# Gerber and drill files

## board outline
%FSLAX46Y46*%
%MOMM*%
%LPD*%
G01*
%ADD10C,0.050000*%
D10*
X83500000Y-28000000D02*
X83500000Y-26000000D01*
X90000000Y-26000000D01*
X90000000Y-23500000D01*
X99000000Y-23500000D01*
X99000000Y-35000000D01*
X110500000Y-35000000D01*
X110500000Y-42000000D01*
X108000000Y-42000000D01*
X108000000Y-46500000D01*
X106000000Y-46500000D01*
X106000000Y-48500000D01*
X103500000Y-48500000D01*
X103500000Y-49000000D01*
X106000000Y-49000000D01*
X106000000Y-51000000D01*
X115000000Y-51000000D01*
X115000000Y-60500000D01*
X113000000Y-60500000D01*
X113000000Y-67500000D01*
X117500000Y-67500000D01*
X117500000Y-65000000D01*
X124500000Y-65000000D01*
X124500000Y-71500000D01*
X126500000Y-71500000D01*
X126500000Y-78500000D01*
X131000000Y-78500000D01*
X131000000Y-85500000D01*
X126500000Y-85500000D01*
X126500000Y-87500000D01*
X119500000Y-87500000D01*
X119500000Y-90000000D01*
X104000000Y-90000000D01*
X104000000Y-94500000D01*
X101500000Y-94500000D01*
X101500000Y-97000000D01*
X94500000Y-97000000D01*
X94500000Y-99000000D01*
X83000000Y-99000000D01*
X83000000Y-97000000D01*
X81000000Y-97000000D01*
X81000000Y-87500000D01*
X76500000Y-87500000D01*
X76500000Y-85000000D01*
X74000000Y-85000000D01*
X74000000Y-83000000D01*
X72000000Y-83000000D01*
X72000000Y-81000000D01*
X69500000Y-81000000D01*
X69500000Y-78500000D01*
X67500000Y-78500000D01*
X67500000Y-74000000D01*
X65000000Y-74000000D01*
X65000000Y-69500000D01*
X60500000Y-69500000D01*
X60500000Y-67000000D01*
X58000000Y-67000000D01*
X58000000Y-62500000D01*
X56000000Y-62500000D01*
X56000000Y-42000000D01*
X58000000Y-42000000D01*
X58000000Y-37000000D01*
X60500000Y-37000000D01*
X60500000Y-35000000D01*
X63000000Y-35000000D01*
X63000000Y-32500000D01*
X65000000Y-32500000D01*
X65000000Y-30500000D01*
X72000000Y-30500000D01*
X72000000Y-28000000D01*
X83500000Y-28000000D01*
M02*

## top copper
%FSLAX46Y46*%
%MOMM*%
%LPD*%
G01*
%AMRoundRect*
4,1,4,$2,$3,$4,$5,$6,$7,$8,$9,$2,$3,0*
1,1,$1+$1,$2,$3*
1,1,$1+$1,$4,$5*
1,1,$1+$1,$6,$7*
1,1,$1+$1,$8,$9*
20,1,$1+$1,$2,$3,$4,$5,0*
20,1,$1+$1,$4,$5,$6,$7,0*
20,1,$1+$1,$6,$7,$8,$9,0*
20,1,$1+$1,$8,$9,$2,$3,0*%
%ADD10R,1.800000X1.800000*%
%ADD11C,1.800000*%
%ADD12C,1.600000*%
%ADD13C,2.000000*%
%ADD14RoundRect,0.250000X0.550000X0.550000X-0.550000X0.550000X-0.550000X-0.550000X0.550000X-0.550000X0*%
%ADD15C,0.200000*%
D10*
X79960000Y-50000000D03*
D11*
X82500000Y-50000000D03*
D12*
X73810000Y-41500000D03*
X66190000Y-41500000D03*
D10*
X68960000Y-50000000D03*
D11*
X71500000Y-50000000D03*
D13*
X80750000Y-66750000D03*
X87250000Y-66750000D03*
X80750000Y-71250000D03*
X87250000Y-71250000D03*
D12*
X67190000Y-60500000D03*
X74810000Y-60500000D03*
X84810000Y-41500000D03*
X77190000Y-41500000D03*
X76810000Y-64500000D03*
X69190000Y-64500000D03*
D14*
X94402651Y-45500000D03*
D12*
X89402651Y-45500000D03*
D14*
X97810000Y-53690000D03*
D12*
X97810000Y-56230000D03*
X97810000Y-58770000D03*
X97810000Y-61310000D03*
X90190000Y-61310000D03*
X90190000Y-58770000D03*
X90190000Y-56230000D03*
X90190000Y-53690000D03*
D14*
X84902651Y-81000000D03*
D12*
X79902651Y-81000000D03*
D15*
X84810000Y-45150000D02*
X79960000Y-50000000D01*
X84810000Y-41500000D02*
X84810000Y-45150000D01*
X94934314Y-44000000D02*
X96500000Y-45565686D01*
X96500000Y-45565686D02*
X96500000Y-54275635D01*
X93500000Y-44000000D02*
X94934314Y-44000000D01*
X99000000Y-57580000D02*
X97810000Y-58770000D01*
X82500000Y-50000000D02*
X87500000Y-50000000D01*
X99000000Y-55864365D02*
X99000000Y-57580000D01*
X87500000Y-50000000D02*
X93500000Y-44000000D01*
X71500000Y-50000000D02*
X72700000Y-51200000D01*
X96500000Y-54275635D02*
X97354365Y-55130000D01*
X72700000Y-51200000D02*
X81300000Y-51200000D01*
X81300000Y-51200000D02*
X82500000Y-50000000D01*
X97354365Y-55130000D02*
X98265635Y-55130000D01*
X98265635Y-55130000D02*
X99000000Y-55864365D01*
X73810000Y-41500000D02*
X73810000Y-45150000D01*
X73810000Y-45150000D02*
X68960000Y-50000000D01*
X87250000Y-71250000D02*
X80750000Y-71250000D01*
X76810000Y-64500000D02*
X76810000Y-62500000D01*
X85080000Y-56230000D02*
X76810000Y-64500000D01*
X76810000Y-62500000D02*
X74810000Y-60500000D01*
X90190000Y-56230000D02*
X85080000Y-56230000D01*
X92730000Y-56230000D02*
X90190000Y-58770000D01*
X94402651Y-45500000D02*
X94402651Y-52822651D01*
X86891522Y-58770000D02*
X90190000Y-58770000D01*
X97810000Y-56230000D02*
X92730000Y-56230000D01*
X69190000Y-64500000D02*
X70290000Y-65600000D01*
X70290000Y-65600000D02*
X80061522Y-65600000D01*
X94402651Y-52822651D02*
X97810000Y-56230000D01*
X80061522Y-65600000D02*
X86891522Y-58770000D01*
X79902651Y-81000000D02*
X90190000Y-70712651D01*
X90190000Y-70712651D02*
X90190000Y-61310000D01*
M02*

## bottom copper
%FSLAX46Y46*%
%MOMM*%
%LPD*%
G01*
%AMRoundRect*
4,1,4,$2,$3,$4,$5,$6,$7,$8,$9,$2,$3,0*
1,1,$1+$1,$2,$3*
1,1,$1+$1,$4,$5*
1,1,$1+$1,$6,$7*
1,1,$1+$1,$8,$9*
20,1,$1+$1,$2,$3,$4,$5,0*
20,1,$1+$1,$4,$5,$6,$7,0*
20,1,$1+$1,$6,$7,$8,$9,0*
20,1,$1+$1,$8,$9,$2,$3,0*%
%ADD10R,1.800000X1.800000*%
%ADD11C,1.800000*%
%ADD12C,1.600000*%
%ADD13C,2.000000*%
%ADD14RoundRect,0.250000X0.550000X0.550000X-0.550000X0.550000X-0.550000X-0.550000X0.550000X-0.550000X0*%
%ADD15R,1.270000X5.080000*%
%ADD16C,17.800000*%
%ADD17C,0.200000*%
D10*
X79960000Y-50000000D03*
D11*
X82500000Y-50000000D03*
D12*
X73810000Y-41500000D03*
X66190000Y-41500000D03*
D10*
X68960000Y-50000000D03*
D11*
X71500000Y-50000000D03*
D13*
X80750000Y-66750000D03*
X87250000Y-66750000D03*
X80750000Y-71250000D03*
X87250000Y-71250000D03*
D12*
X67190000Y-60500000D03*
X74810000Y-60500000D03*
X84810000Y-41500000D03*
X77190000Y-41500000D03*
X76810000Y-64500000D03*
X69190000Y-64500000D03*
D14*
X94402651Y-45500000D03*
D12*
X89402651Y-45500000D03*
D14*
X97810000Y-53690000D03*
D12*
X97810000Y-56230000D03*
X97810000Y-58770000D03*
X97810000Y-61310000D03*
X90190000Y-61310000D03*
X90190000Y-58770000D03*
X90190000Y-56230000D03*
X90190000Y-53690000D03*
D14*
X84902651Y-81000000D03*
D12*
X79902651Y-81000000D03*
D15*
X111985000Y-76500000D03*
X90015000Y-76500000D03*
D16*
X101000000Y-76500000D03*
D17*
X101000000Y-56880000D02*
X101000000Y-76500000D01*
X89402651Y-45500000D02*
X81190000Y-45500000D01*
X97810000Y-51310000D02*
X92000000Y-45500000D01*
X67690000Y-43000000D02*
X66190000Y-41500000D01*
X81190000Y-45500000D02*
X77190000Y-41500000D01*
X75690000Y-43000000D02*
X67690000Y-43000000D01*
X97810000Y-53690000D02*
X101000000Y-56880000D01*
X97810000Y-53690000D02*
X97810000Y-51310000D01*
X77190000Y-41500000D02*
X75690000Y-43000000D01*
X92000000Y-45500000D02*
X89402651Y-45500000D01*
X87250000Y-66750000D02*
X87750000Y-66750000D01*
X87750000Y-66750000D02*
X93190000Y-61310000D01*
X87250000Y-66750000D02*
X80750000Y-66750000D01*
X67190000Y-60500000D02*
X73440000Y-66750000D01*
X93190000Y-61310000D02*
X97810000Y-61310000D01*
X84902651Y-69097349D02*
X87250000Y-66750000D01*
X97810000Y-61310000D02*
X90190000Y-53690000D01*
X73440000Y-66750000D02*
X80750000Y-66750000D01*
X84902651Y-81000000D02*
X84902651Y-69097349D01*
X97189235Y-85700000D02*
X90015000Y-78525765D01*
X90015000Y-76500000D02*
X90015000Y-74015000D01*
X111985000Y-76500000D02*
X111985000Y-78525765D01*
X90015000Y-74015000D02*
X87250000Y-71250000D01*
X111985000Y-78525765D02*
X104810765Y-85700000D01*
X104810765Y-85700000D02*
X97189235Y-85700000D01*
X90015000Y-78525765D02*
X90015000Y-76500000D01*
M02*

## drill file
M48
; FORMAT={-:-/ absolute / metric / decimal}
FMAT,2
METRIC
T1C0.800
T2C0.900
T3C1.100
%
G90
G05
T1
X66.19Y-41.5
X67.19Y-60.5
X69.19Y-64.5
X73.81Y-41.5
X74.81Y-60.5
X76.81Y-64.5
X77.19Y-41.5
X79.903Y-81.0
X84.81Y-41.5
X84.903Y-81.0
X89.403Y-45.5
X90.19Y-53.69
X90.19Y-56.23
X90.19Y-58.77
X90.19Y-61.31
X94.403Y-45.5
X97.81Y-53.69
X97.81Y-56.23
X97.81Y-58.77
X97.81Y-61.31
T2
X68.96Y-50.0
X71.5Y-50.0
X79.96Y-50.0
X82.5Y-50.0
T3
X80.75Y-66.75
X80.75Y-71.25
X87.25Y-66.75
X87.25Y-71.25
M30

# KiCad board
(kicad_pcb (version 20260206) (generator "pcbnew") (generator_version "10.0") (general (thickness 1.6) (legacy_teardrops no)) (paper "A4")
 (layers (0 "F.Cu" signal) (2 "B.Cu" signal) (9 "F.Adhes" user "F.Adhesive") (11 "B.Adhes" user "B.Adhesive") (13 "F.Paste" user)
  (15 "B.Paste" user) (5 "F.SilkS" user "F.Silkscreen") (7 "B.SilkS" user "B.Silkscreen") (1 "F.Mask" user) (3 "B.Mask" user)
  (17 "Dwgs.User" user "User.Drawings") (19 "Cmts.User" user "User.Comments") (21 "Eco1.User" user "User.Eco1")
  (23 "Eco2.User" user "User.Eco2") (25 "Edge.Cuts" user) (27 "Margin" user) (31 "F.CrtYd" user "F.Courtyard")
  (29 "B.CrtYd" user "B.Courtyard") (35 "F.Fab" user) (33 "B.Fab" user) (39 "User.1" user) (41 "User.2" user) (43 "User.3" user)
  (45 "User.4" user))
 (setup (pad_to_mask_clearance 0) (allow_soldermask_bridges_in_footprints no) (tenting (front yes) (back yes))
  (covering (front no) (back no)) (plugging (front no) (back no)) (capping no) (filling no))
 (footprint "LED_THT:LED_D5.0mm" (layer "F.Cu") (at 79.96 50)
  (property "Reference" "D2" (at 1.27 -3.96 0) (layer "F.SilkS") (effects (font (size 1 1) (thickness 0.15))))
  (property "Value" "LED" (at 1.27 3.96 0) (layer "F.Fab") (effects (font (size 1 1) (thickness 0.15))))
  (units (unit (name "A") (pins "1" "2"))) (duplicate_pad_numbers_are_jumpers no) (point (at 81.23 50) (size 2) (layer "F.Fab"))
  (pad "1" thru_hole rect (at 0 0) (size 1.8 1.8) (drill 0.9) (layers "*.Cu" "*.Mask") (remove_unused_layers no) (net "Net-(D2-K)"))
  (pad "2" thru_hole circle (at 2.54 0) (size 1.8 1.8) (drill 0.9) (layers "*.Cu" "*.Mask") (remove_unused_layers no) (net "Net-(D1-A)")))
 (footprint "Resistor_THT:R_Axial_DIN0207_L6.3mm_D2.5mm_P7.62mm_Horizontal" (layer "F.Cu") (at 73.81 41.5 180)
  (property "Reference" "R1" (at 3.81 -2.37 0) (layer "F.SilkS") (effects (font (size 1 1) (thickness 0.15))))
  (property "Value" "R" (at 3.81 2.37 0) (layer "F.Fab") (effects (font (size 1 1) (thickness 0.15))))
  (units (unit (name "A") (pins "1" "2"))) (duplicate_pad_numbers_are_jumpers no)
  (pad "1" thru_hole circle (at 0 0 180) (size 1.6 1.6) (drill 0.8) (layers "*.Cu" "*.Mask") (remove_unused_layers no) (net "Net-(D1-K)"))
  (pad "2" thru_hole circle (at 7.62 0 180) (size 1.6 1.6) (drill 0.8) (layers "*.Cu" "*.Mask") (remove_unused_layers no)
   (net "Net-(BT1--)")))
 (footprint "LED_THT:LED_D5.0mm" (layer "F.Cu") (at 68.96 50)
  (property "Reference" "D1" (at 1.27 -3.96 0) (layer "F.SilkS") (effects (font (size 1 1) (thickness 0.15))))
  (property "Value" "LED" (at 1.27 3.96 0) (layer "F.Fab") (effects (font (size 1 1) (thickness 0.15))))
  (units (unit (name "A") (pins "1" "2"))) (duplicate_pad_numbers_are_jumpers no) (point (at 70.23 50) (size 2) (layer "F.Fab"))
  (pad "1" thru_hole rect (at 0 0) (size 1.8 1.8) (drill 0.9) (layers "*.Cu" "*.Mask") (remove_unused_layers no) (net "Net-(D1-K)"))
  (pad "2" thru_hole circle (at 2.54 0) (size 1.8 1.8) (drill 0.9) (layers "*.Cu" "*.Mask") (remove_unused_layers no) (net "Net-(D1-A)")))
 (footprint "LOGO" (layer "F.Cu") (at 93.5 61.5)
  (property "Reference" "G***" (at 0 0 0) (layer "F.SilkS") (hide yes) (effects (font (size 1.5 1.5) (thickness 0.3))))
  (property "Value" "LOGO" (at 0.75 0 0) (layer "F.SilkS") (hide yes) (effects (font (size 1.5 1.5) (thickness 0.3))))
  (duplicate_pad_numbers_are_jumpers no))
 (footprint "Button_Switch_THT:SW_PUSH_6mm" (layer "F.Cu") (at 80.75 66.75)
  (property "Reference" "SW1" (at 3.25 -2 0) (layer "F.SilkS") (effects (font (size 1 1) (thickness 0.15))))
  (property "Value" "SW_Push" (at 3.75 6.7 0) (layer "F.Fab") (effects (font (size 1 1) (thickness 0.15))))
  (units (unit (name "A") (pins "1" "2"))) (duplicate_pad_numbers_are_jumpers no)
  (pad "1" thru_hole circle (at 0 0 90) (size 2 2) (drill 1.1) (layers "*.Cu" "*.Mask") (remove_unused_layers no) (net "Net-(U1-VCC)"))
  (pad "1" thru_hole circle (at 6.5 0 90) (size 2 2) (drill 1.1) (layers "*.Cu" "*.Mask") (remove_unused_layers no) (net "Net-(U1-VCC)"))
  (pad "2" thru_hole circle (at 0 4.5 90) (size 2 2) (drill 1.1) (layers "*.Cu" "*.Mask") (remove_unused_layers no) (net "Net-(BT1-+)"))
  (pad "2" thru_hole circle (at 6.5 4.5 90) (size 2 2) (drill 1.1) (layers "*.Cu" "*.Mask") (remove_unused_layers no) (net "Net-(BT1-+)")))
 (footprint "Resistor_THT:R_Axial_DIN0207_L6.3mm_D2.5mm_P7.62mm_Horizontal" (layer "F.Cu") (at 67.19 60.5)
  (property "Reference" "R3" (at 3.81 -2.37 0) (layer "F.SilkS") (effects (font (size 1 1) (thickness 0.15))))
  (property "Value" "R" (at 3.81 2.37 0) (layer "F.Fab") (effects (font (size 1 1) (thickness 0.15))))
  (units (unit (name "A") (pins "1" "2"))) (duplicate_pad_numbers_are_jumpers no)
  (pad "1" thru_hole circle (at 0 0) (size 1.6 1.6) (drill 0.8) (layers "*.Cu" "*.Mask") (remove_unused_layers no) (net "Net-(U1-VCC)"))
  (pad "2" thru_hole circle (at 7.62 0) (size 1.6 1.6) (drill 0.8) (layers "*.Cu" "*.Mask") (remove_unused_layers no) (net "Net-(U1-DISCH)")))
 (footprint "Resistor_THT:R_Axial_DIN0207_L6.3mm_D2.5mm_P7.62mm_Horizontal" (layer "F.Cu") (at 84.81 41.5 180)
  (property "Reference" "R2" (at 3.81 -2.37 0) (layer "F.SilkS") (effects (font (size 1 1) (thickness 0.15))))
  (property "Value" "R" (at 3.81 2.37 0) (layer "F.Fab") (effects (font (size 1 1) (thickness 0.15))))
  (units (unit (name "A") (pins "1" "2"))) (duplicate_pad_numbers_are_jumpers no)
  (pad "1" thru_hole circle (at 0 0 180) (size 1.6 1.6) (drill 0.8) (layers "*.Cu" "*.Mask") (remove_unused_layers no) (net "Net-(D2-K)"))
  (pad "2" thru_hole circle (at 7.62 0 180) (size 1.6 1.6) (drill 0.8) (layers "*.Cu" "*.Mask") (remove_unused_layers no)
   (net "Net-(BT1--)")))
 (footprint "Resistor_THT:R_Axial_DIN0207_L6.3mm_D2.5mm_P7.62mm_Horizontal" (layer "B.Cu") (at 76.81 64.5 180)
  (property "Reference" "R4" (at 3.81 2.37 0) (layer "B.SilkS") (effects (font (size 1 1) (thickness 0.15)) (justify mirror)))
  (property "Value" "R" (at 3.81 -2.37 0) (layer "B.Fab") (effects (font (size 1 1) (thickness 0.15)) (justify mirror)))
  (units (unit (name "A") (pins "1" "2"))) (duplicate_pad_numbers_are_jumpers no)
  (pad "1" thru_hole circle (at 0 0 180) (size 1.6 1.6) (drill 0.8) (layers "*.Cu" "*.Mask") (remove_unused_layers no)
   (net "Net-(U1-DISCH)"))
  (pad "2" thru_hole circle (at 7.62 0 180) (size 1.6 1.6) (drill 0.8) (layers "*.Cu" "*.Mask") (remove_unused_layers no)
   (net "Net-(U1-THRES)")))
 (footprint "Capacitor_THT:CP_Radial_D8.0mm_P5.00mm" (layer "B.Cu") (at 94.402651 45.5 180)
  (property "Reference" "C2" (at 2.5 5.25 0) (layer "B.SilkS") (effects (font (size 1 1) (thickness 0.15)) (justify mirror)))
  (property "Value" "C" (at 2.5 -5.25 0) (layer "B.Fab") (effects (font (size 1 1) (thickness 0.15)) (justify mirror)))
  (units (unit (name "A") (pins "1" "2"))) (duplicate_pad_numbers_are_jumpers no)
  (pad "1" thru_hole roundrect (at 0 0 180) (size 1.6 1.6) (drill 0.8) (layers "*.Cu" "*.Mask") (remove_unused_layers no)
   (roundrect_rratio 0.15625) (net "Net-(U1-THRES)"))
  (pad "2" thru_hole circle (at 5 0 180) (size 1.6 1.6) (drill 0.8) (layers "*.Cu" "*.Mask") (remove_unused_layers no) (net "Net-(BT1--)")))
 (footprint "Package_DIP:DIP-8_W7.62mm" (layer "B.Cu") (at 97.81 53.69 180)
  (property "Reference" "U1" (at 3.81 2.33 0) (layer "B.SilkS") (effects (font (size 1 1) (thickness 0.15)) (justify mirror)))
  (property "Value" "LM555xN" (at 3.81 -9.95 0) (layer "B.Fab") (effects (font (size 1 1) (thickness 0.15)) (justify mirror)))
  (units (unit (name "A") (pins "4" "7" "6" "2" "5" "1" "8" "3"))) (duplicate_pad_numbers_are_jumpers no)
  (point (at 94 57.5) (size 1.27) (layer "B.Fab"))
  (pad "1" thru_hole roundrect (at 0 0 180) (size 1.6 1.6) (drill 0.8) (layers "*.Cu" "*.Mask") (remove_unused_layers no)
   (roundrect_rratio 0.15625) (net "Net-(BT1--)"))
  (pad "2" thru_hole circle (at 0 -2.54 180) (size 1.6 1.6) (drill 0.8) (layers "*.Cu" "*.Mask") (remove_unused_layers no)
   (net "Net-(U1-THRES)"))
  (pad "3" thru_hole circle (at 0 -5.08 180) (size 1.6 1.6) (drill 0.8) (layers "*.Cu" "*.Mask") (remove_unused_layers no)
   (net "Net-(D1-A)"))
  (pad "4" thru_hole circle (at 0 -7.62 180) (size 1.6 1.6) (drill 0.8) (layers "*.Cu" "*.Mask") (remove_unused_layers no)
   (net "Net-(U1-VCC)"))
  (pad "5" thru_hole circle (at 7.62 -7.62 180) (size 1.6 1.6) (drill 0.8) (layers "*.Cu" "*.Mask") (remove_unused_layers no)
   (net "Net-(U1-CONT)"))
  (pad "6" thru_hole circle (at 7.62 -5.08 180) (size 1.6 1.6) (drill 0.8) (layers "*.Cu" "*.Mask") (remove_unused_layers no)
   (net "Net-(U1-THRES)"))
  (pad "7" thru_hole circle (at 7.62 -2.54 180) (size 1.6 1.6) (drill 0.8) (layers "*.Cu" "*.Mask") (remove_unused_layers no)
   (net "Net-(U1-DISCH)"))
  (pad "8" thru_hole circle (at 7.62 0 180) (size 1.6 1.6) (drill 0.8) (layers "*.Cu" "*.Mask") (remove_unused_layers no)
   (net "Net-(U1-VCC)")))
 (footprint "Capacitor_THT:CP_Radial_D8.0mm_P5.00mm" (layer "B.Cu") (at 84.902651 81 180)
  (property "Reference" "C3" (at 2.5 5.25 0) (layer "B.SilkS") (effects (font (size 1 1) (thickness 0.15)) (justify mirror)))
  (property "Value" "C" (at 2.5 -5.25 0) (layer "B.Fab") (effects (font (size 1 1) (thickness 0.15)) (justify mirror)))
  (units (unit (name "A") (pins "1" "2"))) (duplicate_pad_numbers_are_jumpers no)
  (pad "1" thru_hole roundrect (at 0 0 180) (size 1.6 1.6) (drill 0.8) (layers "*.Cu" "*.Mask") (remove_unused_layers no)
   (roundrect_rratio 0.15625) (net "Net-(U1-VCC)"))
  (pad "2" thru_hole circle (at 5 0 180) (size 1.6 1.6) (drill 0.8) (layers "*.Cu" "*.Mask") (remove_unused_layers no) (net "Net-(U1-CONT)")))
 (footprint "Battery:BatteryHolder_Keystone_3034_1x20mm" (layer "B.Cu") (at 101 76.5 180)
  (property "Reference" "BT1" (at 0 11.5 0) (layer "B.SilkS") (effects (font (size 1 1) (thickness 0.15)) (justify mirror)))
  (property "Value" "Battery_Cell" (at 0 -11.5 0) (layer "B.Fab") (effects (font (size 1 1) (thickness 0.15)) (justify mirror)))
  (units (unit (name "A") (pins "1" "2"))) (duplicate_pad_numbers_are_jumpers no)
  (pad "1" smd rect (at -10.985 0 180) (size 1.27 5.08) (layers "B.Cu" "B.Mask" "B.Paste") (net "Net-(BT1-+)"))
  (pad "1" smd rect (at 10.985 0 180) (size 1.27 5.08) (layers "B.Cu" "B.Mask" "B.Paste") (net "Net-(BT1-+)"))
  (pad "2" smd circle (at 0 0 180) (size 17.8 17.8) (layers "B.Cu" "B.Mask") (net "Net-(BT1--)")))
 (gr_poly
  (pts (xy 83.5 28) (xy 83.5 26) (xy 90 26) (xy 90 23.5) (xy 99 23.5) (xy 99 35) (xy 110.5 35) (xy 110.5 42) (xy 108 42) (xy 108 46.5)
   (xy 106 46.5) (xy 106 48.5) (xy 103.5 48.5) (xy 103.5 49) (xy 106 49) (xy 106 51) (xy 115 51) (xy 115 60.5) (xy 113 60.5) (xy 113 67.5)
   (xy 117.5 67.5) (xy 117.5 65) (xy 124.5 65) (xy 124.5 71.5) (xy 126.5 71.5) (xy 126.5 78.5) (xy 131 78.5) (xy 131 85.5) (xy 126.5 85.5)
   (xy 126.5 87.5) (xy 119.5 87.5) (xy 119.5 90) (xy 104 90) (xy 104 94.5) (xy 101.5 94.5) (xy 101.5 97) (xy 94.5 97) (xy 94.5 99)
   (xy 83 99) (xy 83 97) (xy 81 97) (xy 81 87.5) (xy 76.5 87.5) (xy 76.5 85) (xy 74 85) (xy 74 83) (xy 72 83) (xy 72 81) (xy 69.5 81)
   (xy 69.5 78.5) (xy 67.5 78.5) (xy 67.5 74) (xy 65 74) (xy 65 69.5) (xy 60.5 69.5) (xy 60.5 67) (xy 58 67) (xy 58 62.5) (xy 56 62.5)
   (xy 56 42) (xy 58 42) (xy 58 37) (xy 60.5 37) (xy 60.5 35) (xy 63 35) (xy 63 32.5) (xy 65 32.5) (xy 65 30.5) (xy 72 30.5) (xy 72 28))
  (stroke (width 0.05) (type solid)) (fill no) (layer "Edge.Cuts"))
 (segment (start 84.81 45.15) (end 79.96 50) (width 0.2) (layer "F.Cu") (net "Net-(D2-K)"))
 (segment (start 84.81 41.5) (end 84.81 45.15) (width 0.2) (layer "F.Cu") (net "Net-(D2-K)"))
 (segment (start 94.934314 44) (end 96.5 45.565686) (width 0.2) (layer "F.Cu") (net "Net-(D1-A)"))
 (segment (start 96.5 45.565686) (end 96.5 54.275635) (width 0.2) (layer "F.Cu") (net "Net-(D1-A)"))
 (segment (start 93.5 44) (end 94.934314 44) (width 0.2) (layer "F.Cu") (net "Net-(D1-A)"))
 (segment (start 99 57.58) (end 97.81 58.77) (width 0.2) (layer "F.Cu") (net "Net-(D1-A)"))
 (segment (start 82.5 50) (end 87.5 50) (width 0.2) (layer "F.Cu") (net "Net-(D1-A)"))
 (segment (start 99 55.864365) (end 99 57.58) (width 0.2) (layer "F.Cu") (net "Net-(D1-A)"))
 (segment (start 87.5 50) (end 93.5 44) (width 0.2) (layer "F.Cu") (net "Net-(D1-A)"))
 (segment (start 71.5 50) (end 72.7 51.2) (width 0.2) (layer "F.Cu") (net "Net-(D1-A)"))
 (segment (start 96.5 54.275635) (end 97.354365 55.13) (width 0.2) (layer "F.Cu") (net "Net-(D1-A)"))
 (segment (start 72.7 51.2) (end 81.3 51.2) (width 0.2) (layer "F.Cu") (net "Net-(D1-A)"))
 (segment (start 81.3 51.2) (end 82.5 50) (width 0.2) (layer "F.Cu") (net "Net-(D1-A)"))
 (segment (start 97.354365 55.13) (end 98.265635 55.13) (width 0.2) (layer "F.Cu") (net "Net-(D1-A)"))
 (segment (start 98.265635 55.13) (end 99 55.864365) (width 0.2) (layer "F.Cu") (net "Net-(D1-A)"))
 (segment (start 73.81 41.5) (end 73.81 45.15) (width 0.2) (layer "F.Cu") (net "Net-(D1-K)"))
 (segment (start 73.81 45.15) (end 68.96 50) (width 0.2) (layer "F.Cu") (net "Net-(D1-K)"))
 (segment (start 101 56.88) (end 101 76.5) (width 0.2) (layer "B.Cu") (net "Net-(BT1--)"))
 (segment (start 89.402651 45.5) (end 81.19 45.5) (width 0.2) (layer "B.Cu") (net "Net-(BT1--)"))
 (segment (start 97.81 51.31) (end 92 45.5) (width 0.2) (layer "B.Cu") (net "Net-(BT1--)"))
 (segment (start 67.69 43) (end 66.19 41.5) (width 0.2) (layer "B.Cu") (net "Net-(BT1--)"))
 (segment (start 81.19 45.5) (end 77.19 41.5) (width 0.2) (layer "B.Cu") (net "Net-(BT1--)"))
 (segment (start 75.69 43) (end 67.69 43) (width 0.2) (layer "B.Cu") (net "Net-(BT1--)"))
 (segment (start 97.81 53.69) (end 101 56.88) (width 0.2) (layer "B.Cu") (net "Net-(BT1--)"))
 (segment (start 97.81 53.69) (end 97.81 51.31) (width 0.2) (layer "B.Cu") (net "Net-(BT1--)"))
 (segment (start 77.19 41.5) (end 75.69 43) (width 0.2) (layer "B.Cu") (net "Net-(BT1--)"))
 (segment (start 92 45.5) (end 89.402651 45.5) (width 0.2) (layer "B.Cu") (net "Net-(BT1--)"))
 (segment (start 87.25 66.75) (end 87.75 66.75) (width 0.2) (layer "B.Cu") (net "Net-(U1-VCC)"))
 (segment (start 87.75 66.75) (end 93.19 61.31) (width 0.2) (layer "B.Cu") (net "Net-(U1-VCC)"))
 (segment (start 87.25 66.75) (end 80.75 66.75) (width 0.2) (layer "B.Cu") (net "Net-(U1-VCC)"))
 (segment (start 67.19 60.5) (end 73.44 66.75) (width 0.2) (layer "B.Cu") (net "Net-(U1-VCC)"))
 (segment (start 93.19 61.31) (end 97.81 61.31) (width 0.2) (layer "B.Cu") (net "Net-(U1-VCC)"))
 (segment (start 84.902651 69.097349) (end 87.25 66.75) (width 0.2) (layer "B.Cu") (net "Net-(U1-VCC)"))
 (segment (start 97.81 61.31) (end 90.19 53.69) (width 0.2) (layer "B.Cu") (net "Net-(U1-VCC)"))
 (segment (start 73.44 66.75) (end 80.75 66.75) (width 0.2) (layer "B.Cu") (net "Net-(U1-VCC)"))
 (segment (start 84.902651 81) (end 84.902651 69.097349) (width 0.2) (layer "B.Cu") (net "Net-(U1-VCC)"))
 (segment (start 87.25 71.25) (end 80.75 71.25) (width 0.2) (layer "F.Cu") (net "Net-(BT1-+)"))
 (segment (start 97.189235 85.7) (end 90.015 78.525765) (width 0.2) (layer "B.Cu") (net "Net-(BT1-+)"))
 (segment (start 90.015 76.5) (end 90.015 74.015) (width 0.2) (layer "B.Cu") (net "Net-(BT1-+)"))
 (segment (start 111.985 76.5) (end 111.985 78.525765) (width 0.2) (layer "B.Cu") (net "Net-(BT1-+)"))
 (segment (start 90.015 74.015) (end 87.25 71.25) (width 0.2) (layer "B.Cu") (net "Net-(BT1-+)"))
 (segment (start 111.985 78.525765) (end 104.810765 85.7) (width 0.2) (layer "B.Cu") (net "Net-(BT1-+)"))
 (segment (start 104.810765 85.7) (end 97.189235 85.7) (width 0.2) (layer "B.Cu") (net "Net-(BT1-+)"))
 (segment (start 90.015 78.525765) (end 90.015 76.5) (width 0.2) (layer "B.Cu") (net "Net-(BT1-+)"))
 (segment (start 76.81 64.5) (end 76.81 62.5) (width 0.2) (layer "F.Cu") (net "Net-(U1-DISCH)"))
 (segment (start 85.08 56.23) (end 76.81 64.5) (width 0.2) (layer "F.Cu") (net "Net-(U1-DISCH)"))
 (segment (start 76.81 62.5) (end 74.81 60.5) (width 0.2) (layer "F.Cu") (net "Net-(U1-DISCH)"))
 (segment (start 90.19 56.23) (end 85.08 56.23) (width 0.2) (layer "F.Cu") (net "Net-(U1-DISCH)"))
 (segment (start 92.73 56.23) (end 90.19 58.77) (width 0.2) (layer "F.Cu") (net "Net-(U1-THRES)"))
 (segment (start 94.402651 45.5) (end 94.402651 52.822651) (width 0.2) (layer "F.Cu") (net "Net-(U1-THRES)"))
 (segment (start 86.891522 58.77) (end 90.19 58.77) (width 0.2) (layer "F.Cu") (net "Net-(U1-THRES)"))
 (segment (start 97.81 56.23) (end 92.73 56.23) (width 0.2) (layer "F.Cu") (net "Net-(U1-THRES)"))
 (segment (start 69.19 64.5) (end 70.29 65.6) (width 0.2) (layer "F.Cu") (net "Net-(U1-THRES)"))
 (segment (start 70.29 65.6) (end 80.061522 65.6) (width 0.2) (layer "F.Cu") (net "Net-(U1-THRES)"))
 (segment (start 94.402651 52.822651) (end 97.81 56.23) (width 0.2) (layer "F.Cu") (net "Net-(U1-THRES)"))
 (segment (start 80.061522 65.6) (end 86.891522 58.77) (width 0.2) (layer "F.Cu") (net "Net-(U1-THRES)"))
 (segment (start 79.902651 81) (end 90.19 70.712651) (width 0.2) (layer "F.Cu") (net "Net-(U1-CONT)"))
 (segment (start 90.19 70.712651) (end 90.19 61.31) (width 0.2) (layer "F.Cu") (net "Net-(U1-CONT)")))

